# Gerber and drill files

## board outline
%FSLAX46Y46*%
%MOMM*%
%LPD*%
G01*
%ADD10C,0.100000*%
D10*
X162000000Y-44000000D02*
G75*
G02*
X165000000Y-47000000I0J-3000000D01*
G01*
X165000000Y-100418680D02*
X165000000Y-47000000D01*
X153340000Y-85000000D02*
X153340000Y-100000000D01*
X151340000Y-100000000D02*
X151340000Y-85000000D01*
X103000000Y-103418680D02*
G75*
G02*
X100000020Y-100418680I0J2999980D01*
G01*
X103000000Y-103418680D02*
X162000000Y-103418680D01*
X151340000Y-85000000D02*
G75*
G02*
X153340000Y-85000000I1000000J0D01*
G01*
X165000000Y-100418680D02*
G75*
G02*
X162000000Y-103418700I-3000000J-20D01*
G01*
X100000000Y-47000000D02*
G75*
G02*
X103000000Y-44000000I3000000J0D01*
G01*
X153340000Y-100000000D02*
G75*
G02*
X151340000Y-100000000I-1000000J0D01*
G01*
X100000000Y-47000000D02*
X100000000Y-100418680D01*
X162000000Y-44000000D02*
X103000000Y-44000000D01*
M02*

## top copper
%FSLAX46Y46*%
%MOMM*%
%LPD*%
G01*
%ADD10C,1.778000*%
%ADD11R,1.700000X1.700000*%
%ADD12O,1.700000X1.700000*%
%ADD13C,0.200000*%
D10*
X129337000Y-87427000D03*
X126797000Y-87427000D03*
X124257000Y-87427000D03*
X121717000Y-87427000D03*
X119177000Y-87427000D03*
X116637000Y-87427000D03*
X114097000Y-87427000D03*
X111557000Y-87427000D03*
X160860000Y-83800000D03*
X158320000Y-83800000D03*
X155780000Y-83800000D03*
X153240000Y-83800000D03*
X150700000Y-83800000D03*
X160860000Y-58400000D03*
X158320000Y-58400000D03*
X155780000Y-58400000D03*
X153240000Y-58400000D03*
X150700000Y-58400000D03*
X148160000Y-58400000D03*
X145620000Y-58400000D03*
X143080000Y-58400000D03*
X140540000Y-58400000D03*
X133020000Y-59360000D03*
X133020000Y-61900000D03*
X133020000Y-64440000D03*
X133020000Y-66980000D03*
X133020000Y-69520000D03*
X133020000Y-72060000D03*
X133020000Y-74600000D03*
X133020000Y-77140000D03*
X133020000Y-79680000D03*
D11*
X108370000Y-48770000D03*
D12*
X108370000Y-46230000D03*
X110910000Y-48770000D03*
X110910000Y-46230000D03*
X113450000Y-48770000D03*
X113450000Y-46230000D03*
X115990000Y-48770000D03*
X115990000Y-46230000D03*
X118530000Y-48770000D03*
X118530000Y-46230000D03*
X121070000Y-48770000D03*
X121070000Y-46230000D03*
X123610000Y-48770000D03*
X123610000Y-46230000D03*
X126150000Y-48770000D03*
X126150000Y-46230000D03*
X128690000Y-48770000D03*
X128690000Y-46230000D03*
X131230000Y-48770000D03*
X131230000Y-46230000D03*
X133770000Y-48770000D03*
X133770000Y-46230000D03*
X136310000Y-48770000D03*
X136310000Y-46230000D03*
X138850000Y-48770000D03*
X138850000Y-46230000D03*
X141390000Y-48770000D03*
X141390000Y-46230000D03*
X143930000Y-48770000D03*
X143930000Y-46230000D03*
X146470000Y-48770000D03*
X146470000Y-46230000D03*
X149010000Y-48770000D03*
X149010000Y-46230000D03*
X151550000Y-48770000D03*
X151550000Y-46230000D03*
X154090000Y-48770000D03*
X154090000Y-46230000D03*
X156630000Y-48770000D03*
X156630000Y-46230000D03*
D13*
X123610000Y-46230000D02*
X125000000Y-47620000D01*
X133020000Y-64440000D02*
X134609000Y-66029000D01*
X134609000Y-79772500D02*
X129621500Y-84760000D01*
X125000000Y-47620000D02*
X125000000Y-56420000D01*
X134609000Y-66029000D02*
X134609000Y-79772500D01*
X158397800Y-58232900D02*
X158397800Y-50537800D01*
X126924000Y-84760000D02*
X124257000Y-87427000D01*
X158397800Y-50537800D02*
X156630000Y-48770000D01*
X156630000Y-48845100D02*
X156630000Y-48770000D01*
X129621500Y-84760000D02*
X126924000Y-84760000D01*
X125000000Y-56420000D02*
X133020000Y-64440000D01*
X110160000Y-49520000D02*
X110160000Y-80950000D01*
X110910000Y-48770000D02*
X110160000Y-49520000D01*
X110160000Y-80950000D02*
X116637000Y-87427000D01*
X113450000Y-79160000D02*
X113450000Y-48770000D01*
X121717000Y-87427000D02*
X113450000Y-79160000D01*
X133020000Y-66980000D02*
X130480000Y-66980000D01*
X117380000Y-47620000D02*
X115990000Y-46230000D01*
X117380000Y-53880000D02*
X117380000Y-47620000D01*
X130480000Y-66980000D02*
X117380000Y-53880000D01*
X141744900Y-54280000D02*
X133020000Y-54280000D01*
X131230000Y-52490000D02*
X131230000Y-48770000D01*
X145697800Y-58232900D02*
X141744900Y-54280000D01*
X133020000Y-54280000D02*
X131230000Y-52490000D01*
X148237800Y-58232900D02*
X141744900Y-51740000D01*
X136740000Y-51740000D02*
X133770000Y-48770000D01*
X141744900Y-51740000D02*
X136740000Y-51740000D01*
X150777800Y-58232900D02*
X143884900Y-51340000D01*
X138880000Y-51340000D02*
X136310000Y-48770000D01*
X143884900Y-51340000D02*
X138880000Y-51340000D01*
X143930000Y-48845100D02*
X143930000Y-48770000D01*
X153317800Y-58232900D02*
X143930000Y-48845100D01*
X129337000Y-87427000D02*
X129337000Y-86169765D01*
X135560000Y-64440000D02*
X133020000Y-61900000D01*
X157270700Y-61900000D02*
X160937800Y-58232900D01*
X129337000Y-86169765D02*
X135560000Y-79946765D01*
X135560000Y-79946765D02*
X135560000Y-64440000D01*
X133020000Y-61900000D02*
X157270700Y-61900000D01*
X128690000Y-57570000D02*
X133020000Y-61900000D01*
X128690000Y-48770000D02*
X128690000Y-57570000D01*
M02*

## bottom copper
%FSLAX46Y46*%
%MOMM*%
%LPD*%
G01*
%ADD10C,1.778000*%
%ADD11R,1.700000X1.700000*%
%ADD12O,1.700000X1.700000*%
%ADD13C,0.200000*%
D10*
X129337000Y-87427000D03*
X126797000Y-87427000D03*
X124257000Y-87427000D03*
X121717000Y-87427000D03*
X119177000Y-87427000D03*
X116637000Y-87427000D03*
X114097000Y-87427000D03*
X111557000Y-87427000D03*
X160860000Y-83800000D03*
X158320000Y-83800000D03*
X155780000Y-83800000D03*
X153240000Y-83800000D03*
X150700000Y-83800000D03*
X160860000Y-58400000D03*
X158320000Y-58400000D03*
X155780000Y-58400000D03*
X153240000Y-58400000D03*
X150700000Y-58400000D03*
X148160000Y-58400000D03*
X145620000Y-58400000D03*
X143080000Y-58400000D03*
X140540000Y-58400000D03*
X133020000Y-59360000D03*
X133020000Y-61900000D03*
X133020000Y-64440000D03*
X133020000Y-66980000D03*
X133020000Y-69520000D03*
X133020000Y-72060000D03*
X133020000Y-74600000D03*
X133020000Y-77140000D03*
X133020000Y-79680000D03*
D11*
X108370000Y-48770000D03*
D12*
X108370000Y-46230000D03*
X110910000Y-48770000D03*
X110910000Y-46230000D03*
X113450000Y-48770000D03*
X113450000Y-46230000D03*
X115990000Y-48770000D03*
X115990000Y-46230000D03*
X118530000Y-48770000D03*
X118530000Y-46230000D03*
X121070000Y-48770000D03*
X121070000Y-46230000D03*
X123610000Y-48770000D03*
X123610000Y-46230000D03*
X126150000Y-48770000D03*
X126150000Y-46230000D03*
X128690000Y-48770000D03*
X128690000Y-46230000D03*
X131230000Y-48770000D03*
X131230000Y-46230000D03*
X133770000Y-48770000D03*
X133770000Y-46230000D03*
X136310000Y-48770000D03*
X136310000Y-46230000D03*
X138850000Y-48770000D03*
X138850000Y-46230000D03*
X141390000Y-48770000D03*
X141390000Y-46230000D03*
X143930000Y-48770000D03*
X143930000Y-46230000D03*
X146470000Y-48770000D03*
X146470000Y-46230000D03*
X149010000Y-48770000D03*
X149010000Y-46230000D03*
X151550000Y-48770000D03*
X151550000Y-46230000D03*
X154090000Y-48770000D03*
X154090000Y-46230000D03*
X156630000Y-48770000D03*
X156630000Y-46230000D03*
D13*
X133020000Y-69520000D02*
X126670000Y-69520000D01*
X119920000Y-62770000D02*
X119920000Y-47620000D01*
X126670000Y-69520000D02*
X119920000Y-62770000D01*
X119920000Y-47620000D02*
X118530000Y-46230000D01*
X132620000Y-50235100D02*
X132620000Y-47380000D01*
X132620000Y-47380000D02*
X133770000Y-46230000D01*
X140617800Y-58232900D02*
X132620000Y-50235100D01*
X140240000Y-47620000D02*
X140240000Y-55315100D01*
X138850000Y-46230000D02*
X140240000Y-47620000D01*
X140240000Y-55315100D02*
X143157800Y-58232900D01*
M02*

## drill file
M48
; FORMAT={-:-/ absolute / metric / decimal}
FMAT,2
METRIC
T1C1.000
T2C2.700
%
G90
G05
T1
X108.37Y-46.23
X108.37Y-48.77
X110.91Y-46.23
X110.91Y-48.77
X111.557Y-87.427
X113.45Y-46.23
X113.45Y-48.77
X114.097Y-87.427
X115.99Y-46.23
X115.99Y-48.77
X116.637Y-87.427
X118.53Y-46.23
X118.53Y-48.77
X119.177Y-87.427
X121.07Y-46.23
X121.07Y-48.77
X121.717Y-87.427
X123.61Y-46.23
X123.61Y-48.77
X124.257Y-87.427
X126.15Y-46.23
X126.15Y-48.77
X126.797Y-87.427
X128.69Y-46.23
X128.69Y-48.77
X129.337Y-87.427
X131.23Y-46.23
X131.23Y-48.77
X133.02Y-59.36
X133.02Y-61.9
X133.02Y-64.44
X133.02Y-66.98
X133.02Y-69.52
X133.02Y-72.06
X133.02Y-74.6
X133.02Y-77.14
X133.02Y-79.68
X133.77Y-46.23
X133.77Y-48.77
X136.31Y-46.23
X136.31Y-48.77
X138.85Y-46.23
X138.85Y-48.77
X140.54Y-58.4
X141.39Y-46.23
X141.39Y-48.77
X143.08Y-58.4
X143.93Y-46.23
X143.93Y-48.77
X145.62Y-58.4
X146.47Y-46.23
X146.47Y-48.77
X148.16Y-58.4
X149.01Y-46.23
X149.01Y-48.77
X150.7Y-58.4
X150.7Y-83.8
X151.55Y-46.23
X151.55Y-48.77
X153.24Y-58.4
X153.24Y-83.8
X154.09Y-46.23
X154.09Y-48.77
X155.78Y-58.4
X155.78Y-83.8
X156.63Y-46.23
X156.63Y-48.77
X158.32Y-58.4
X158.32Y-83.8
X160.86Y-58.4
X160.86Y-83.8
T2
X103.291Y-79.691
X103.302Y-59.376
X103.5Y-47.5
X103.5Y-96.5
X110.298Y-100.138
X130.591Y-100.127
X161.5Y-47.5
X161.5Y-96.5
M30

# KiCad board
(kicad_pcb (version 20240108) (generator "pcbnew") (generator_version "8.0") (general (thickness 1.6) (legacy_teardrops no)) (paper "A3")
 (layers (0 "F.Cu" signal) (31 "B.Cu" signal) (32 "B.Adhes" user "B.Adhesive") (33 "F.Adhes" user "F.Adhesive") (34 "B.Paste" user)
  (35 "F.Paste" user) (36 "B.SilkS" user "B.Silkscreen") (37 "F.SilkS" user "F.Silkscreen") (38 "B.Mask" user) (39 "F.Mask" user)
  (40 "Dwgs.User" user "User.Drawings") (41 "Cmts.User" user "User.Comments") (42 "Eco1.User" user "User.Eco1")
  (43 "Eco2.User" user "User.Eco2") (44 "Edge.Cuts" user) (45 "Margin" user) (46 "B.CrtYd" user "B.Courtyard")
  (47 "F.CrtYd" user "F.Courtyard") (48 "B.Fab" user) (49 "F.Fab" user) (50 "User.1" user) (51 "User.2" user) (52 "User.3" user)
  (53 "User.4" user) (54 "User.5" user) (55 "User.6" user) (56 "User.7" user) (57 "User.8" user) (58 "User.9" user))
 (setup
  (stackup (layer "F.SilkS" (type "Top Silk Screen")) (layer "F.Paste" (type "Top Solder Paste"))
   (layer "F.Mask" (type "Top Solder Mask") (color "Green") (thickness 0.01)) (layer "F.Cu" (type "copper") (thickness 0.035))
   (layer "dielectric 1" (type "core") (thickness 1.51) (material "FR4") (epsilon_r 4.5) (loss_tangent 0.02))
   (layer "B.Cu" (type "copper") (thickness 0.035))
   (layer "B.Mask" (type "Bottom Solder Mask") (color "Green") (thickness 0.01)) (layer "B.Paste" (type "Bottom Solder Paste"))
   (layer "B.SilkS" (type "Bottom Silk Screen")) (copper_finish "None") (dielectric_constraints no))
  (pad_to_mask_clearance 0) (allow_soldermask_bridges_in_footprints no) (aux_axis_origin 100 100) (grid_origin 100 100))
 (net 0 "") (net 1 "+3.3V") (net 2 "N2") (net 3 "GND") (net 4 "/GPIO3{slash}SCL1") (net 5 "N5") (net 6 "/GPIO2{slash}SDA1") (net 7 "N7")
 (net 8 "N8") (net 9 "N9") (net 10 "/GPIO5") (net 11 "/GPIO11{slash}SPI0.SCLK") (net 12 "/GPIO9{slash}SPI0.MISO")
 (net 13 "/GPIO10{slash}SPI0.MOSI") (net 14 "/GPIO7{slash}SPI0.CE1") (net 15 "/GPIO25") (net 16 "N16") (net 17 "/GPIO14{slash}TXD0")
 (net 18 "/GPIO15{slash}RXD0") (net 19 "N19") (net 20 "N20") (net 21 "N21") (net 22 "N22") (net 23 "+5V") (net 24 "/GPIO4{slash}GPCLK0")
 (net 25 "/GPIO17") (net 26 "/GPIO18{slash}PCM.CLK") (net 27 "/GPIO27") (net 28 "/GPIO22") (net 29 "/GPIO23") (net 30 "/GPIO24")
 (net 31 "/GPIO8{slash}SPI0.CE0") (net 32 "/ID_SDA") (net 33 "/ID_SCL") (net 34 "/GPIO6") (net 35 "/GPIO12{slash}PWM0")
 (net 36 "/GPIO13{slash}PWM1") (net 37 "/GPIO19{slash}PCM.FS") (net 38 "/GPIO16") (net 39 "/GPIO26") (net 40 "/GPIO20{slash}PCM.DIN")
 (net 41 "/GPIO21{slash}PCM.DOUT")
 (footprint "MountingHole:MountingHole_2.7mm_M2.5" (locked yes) (layer "F.Cu") (at 161.5 47.5)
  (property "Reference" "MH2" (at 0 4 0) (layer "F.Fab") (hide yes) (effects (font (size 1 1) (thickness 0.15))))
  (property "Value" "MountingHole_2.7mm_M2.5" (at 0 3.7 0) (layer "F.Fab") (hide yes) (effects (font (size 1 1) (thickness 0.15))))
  (pad "" np_thru_hole circle (at 0 0) (size 2.7 2.7) (drill 2.7) (layers "*.Cu" "*.Mask")))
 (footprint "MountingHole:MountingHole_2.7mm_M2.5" (layer "F.Cu") (at 103.290686 79.691314)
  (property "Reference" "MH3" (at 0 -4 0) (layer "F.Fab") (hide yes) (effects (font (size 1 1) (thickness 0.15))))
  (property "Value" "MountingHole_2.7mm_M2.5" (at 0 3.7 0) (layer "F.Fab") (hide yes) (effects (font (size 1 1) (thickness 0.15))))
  (pad "" np_thru_hole circle (at 0 0) (size 2.7 2.7) (drill 2.7) (layers "*.Cu" "*.Mask")))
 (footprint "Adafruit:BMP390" (layer "F.Cu") (at 120.32 92.38 180)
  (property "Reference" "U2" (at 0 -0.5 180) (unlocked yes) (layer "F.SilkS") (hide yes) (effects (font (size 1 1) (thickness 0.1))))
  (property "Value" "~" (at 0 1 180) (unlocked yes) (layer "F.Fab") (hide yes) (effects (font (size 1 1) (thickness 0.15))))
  (pad "1" thru_hole circle (at -9.017 4.953 270) (size 1.778 1.778) (drill 1) (layers "*.Cu" "*.Mask") (remove_unused_layers no)
   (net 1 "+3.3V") (solder_mask_margin 0.0508) (thermal_bridge_angle 0))
  (pad "2" thru_hole circle (at -6.477 4.953 270) (size 1.778 1.778) (drill 1) (layers "*.Cu" "*.Mask") (remove_unused_layers no)
   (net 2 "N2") (solder_mask_margin 0.0508) (thermal_bridge_angle 0))
  (pad "3" thru_hole circle (at -3.937 4.953 270) (size 1.778 1.778) (drill 1) (layers "*.Cu" "*.Mask") (remove_unused_layers no)
   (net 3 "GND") (solder_mask_margin 0.0508) (thermal_bridge_angle 0))
  (pad "4" thru_hole circle (at -1.397 4.953 270) (size 1.778 1.778) (drill 1) (layers "*.Cu" "*.Mask") (remove_unused_layers no)
   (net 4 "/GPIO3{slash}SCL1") (solder_mask_margin 0.0508) (thermal_bridge_angle 0))
  (pad "5" thru_hole circle (at 1.143 4.953 270) (size 1.778 1.778) (drill 1) (layers "*.Cu" "*.Mask") (remove_unused_layers no)
   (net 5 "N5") (solder_mask_margin 0.0508) (thermal_bridge_angle 0))
  (pad "6" thru_hole circle (at 3.683 4.953 270) (size 1.778 1.778) (drill 1) (layers "*.Cu" "*.Mask") (remove_unused_layers no)
   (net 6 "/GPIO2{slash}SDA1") (solder_mask_margin 0.0508) (thermal_bridge_angle 0))
  (pad "7" thru_hole circle (at 6.223 4.953 270) (size 1.778 1.778) (drill 1) (layers "*.Cu" "*.Mask") (remove_unused_layers no)
   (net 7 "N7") (solder_mask_margin 0.0508) (thermal_bridge_angle 0))
  (pad "8" thru_hole circle (at 8.763 4.953 270) (size 1.778 1.778) (drill 1) (layers "*.Cu" "*.Mask") (remove_unused_layers no)
   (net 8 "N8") (solder_mask_margin 0.0508) (thermal_bridge_angle 0)))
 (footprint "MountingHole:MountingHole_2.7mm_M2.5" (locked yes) (layer "F.Cu") (at 103.5 96.5)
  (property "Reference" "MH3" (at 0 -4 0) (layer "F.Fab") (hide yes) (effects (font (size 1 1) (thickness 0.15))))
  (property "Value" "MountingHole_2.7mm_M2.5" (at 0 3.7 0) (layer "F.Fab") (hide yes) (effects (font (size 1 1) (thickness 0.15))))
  (pad "" np_thru_hole circle (at 0 0) (size 2.7 2.7) (drill 2.7) (layers "*.Cu" "*.Mask")))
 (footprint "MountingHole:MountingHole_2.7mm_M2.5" (layer "F.Cu") (at 130.591 100.127)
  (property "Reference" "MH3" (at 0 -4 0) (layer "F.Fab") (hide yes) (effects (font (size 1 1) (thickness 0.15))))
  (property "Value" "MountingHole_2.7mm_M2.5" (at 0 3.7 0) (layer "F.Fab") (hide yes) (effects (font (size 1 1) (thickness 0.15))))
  (pad "" np_thru_hole circle (at 0 0) (size 2.7 2.7) (drill 2.7) (layers "*.Cu" "*.Mask")))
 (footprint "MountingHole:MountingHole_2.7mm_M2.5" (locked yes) (layer "F.Cu") (at 103.5 47.5)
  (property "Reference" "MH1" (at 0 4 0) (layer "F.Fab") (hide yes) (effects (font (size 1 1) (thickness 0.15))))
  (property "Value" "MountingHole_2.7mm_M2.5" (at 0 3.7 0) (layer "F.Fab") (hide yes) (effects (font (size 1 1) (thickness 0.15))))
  (pad "" np_thru_hole circle (at 0 0) (size 2.7 2.7) (drill 2.7) (layers "*.Cu" "*.Mask")))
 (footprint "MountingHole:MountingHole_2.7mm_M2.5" (layer "F.Cu") (at 110.298314 100.138314)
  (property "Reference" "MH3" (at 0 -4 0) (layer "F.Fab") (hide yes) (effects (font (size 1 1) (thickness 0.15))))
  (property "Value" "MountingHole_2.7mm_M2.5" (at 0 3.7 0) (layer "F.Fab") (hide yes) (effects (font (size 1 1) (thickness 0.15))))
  (pad "" np_thru_hole circle (at 0 0) (size 2.7 2.7) (drill 2.7) (layers "*.Cu" "*.Mask")))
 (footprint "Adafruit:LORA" (layer "F.Cu") (at 150.7222 69.6871 180)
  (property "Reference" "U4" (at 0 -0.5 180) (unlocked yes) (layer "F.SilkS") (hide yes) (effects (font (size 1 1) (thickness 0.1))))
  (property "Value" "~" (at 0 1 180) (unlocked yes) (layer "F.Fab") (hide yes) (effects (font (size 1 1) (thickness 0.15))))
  (pad "" thru_hole circle (at -10.1378 -14.1129 270) (size 1.778 1.778) (drill 1) (layers "*.Cu" "*.Mask") (remove_unused_layers no)
   (solder_mask_margin 0.0508) (thermal_bridge_angle 0))
  (pad "" thru_hole circle (at -7.5978 -14.1129 270) (size 1.778 1.778) (drill 1) (layers "*.Cu" "*.Mask") (remove_unused_layers no)
   (solder_mask_margin 0.0508) (thermal_bridge_angle 0))
  (pad "" thru_hole circle (at -5.0578 -14.1129 270) (size 1.778 1.778) (drill 1) (layers "*.Cu" "*.Mask") (remove_unused_layers no)
   (solder_mask_margin 0.0508) (thermal_bridge_angle 0))
  (pad "" thru_hole circle (at -2.5178 -14.1129 270) (size 1.778 1.778) (drill 1) (layers "*.Cu" "*.Mask") (remove_unused_layers no)
   (solder_mask_margin 0.0508) (thermal_bridge_angle 0))
  (pad "" thru_hole circle (at 0.0222 -14.1129 270) (size 1.778 1.778) (drill 1) (layers "*.Cu" "*.Mask") (remove_unused_layers no)
   (solder_mask_margin 0.0508) (thermal_bridge_angle 0))
  (pad "1" thru_hole circle (at -10.1378 11.2871 270) (size 1.778 1.778) (drill 1) (layers "*.Cu" "*.Mask") (remove_unused_layers no)
   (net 1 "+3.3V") (solder_mask_margin 0.0508) (thermal_bridge_angle 0))
  (pad "2" thru_hole circle (at -7.5978 11.2871 270) (size 1.778 1.778) (drill 1) (layers "*.Cu" "*.Mask") (remove_unused_layers no)
   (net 3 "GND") (solder_mask_margin 0.0508) (thermal_bridge_angle 0))
  (pad "3" thru_hole circle (at -5.0578 11.2871 270) (size 1.778 1.778) (drill 1) (layers "*.Cu" "*.Mask") (remove_unused_layers no)
   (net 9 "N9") (solder_mask_margin 0.0508) (thermal_bridge_angle 0))
  (pad "4" thru_hole circle (at -2.5178 11.2871 270) (size 1.778 1.778) (drill 1) (layers "*.Cu" "*.Mask") (remove_unused_layers no)
   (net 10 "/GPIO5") (solder_mask_margin 0.0508) (thermal_bridge_angle 0))
  (pad "5" thru_hole circle (at 0.0222 11.2871 270) (size 1.778 1.778) (drill 1) (layers "*.Cu" "*.Mask") (remove_unused_layers no)
   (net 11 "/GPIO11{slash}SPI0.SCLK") (solder_mask_margin 0.0508) (thermal_bridge_angle 0))
  (pad "6" thru_hole circle (at 2.5622 11.2871 270) (size 1.778 1.778) (drill 1) (layers "*.Cu" "*.Mask") (remove_unused_layers no)
   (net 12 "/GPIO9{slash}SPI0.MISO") (solder_mask_margin 0.0508) (thermal_bridge_angle 0))
  (pad "7" thru_hole circle (at 5.1022 11.2871 270) (size 1.778 1.778) (drill 1) (layers "*.Cu" "*.Mask") (remove_unused_layers no)
   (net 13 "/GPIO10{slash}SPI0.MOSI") (solder_mask_margin 0.0508) (thermal_bridge_angle 0))
  (pad "8" thru_hole circle (at 7.6422 11.2871 270) (size 1.778 1.778) (drill 1) (layers "*.Cu" "*.Mask") (remove_unused_layers no)
   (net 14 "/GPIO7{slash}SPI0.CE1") (solder_mask_margin 0.0508) (thermal_bridge_angle 0))
  (pad "9" thru_hole circle (at 10.1822 11.2871 270) (size 1.778 1.778) (drill 1) (layers "*.Cu" "*.Mask") (remove_unused_layers no)
   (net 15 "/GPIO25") (solder_mask_margin 0.0508) (thermal_bridge_angle 0)))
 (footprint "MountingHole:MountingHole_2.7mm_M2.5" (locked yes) (layer "F.Cu") (at 161.5 96.5)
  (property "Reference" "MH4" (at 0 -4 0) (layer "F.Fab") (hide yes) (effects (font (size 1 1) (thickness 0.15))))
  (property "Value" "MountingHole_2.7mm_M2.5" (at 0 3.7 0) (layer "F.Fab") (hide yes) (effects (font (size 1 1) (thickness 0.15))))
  (pad "" np_thru_hole circle (at 0 0) (size 2.7 2.7) (drill 2.7) (layers "*.Cu" "*.Mask")))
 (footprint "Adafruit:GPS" (layer "F.Cu") (at 132.639 69.393 90)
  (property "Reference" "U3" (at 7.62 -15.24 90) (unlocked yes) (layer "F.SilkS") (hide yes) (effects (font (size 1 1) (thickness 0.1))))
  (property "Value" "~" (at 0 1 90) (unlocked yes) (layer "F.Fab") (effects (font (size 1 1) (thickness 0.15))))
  (pad "1" thru_hole circle (at 10.033 0.381) (size 1.778 1.778) (drill 1) (layers "*.Cu" "*.Mask") (remove_unused_layers no) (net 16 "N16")
   (solder_mask_margin 0.0508) (thermal_bridge_angle 0))
  (pad "2" thru_hole circle (at 7.493 0.381) (size 1.778 1.778) (drill 1) (layers "*.Cu" "*.Mask") (remove_unused_layers no) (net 1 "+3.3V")
   (solder_mask_margin 0.0508) (thermal_bridge_angle 0))
  (pad "3" thru_hole circle (at 4.953 0.381) (size 1.778 1.778) (drill 1) (layers "*.Cu" "*.Mask") (remove_unused_layers no) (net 3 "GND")
   (solder_mask_margin 0.0508) (thermal_bridge_angle 0))
  (pad "4" thru_hole circle (at 2.413 0.381) (size 1.778 1.778) (drill 1) (layers "*.Cu" "*.Mask") (remove_unused_layers no)
   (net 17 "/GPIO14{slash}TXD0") (solder_mask_margin 0.0508) (thermal_bridge_angle 0))
  (pad "5" thru_hole circle (at -0.127 0.381) (size 1.778 1.778) (drill 1) (layers "*.Cu" "*.Mask") (remove_unused_layers no)
   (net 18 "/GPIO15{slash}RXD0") (solder_mask_margin 0.0508) (thermal_bridge_angle 0))
  (pad "6" thru_hole circle (at -2.667 0.381) (size 1.778 1.778) (drill 1) (layers "*.Cu" "*.Mask") (remove_unused_layers no) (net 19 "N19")
   (solder_mask_margin 0.0508) (thermal_bridge_angle 0))
  (pad "7" thru_hole circle (at -5.207 0.381) (size 1.778 1.778) (drill 1) (layers "*.Cu" "*.Mask") (remove_unused_layers no) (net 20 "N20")
   (solder_mask_margin 0.0508) (thermal_bridge_angle 0))
  (pad "8" thru_hole circle (at -7.747 0.381) (size 1.778 1.778) (drill 1) (layers "*.Cu" "*.Mask") (remove_unused_layers no) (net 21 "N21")
   (solder_mask_margin 0.0508) (thermal_bridge_angle 0))
  (pad "9" thru_hole circle (at -10.287 0.381) (size 1.778 1.778) (drill 1) (layers "*.Cu" "*.Mask") (remove_unused_layers no)
   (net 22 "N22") (solder_mask_margin 0.0508) (thermal_bridge_angle 0)))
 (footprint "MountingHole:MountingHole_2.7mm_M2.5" (layer "F.Cu") (at 103.302 59.376)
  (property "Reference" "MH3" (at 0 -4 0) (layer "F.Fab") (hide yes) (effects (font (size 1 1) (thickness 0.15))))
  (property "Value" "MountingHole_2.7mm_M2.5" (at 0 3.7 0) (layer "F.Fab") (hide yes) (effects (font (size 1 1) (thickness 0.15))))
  (pad "" np_thru_hole circle (at 0 0) (size 2.7 2.7) (drill 2.7) (layers "*.Cu" "*.Mask")))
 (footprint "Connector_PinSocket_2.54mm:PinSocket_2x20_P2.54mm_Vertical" (layer "B.Cu") (at 108.37 48.77 -90)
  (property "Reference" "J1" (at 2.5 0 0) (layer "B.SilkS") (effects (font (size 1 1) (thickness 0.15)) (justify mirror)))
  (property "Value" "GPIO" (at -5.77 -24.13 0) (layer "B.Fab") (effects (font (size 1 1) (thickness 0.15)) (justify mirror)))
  (pad "1" thru_hole rect (at 0 0 270) (size 1.7 1.7) (drill 1) (layers "*.Cu" "*.Mask") (remove_unused_layers no) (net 1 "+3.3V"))
  (pad "2" thru_hole oval (at -2.54 0 270) (size 1.7 1.7) (drill 1) (layers "*.Cu" "*.Mask") (remove_unused_layers no) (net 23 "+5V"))
  (pad "3" thru_hole oval (at 0 -2.54 270) (size 1.7 1.7) (drill 1) (layers "*.Cu" "*.Mask") (remove_unused_layers no)
   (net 6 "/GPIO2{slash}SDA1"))
  (pad "4" thru_hole oval (at -2.54 -2.54 270) (size 1.7 1.7) (drill 1) (layers "*.Cu" "*.Mask") (remove_unused_layers no) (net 23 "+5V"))
  (pad "5" thru_hole oval (at 0 -5.08 270) (size 1.7 1.7) (drill 1) (layers "*.Cu" "*.Mask") (remove_unused_layers no)
   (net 4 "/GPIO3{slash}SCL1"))
  (pad "6" thru_hole oval (at -2.54 -5.08 270) (size 1.7 1.7) (drill 1) (layers "*.Cu" "*.Mask") (remove_unused_layers no) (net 3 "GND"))
  (pad "7" thru_hole oval (at 0 -7.62 270) (size 1.7 1.7) (drill 1) (layers "*.Cu" "*.Mask") (remove_unused_layers no)
   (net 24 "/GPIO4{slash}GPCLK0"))
  (pad "8" thru_hole oval (at -2.54 -7.62 270) (size 1.7 1.7) (drill 1) (layers "*.Cu" "*.Mask") (remove_unused_layers no)
   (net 17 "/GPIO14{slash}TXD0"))
  (pad "9" thru_hole oval (at 0 -10.16 270) (size 1.7 1.7) (drill 1) (layers "*.Cu" "*.Mask") (remove_unused_layers no) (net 3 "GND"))
  (pad "10" thru_hole oval (at -2.54 -10.16 270) (size 1.7 1.7) (drill 1) (layers "*.Cu" "*.Mask") (remove_unused_layers no)
   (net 18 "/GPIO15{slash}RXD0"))
  (pad "11" thru_hole oval (at 0 -12.7 270) (size 1.7 1.7) (drill 1) (layers "*.Cu" "*.Mask") (remove_unused_layers no) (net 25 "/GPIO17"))
  (pad "12" thru_hole oval (at -2.54 -12.7 270) (size 1.7 1.7) (drill 1) (layers "*.Cu" "*.Mask") (remove_unused_layers no)
   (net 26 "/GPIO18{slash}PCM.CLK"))
  (pad "13" thru_hole oval (at 0 -15.24 270) (size 1.7 1.7) (drill 1) (layers "*.Cu" "*.Mask") (remove_unused_layers no) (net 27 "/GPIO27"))
  (pad "14" thru_hole oval (at -2.54 -15.24 270) (size 1.7 1.7) (drill 1) (layers "*.Cu" "*.Mask") (remove_unused_layers no) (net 3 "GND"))
  (pad "15" thru_hole oval (at 0 -17.78 270) (size 1.7 1.7) (drill 1) (layers "*.Cu" "*.Mask") (remove_unused_layers no) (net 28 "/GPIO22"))
  (pad "16" thru_hole oval (at -2.54 -17.78 270) (size 1.7 1.7) (drill 1) (layers "*.Cu" "*.Mask") (remove_unused_layers no)
   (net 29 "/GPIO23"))
  (pad "17" thru_hole oval (at 0 -20.32 270) (size 1.7 1.7) (drill 1) (layers "*.Cu" "*.Mask") (remove_unused_layers no) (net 1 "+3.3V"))
  (pad "18" thru_hole oval (at -2.54 -20.32 270) (size 1.7 1.7) (drill 1) (layers "*.Cu" "*.Mask") (remove_unused_layers no)
   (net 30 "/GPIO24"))
  (pad "19" thru_hole oval (at 0 -22.86 270) (size 1.7 1.7) (drill 1) (layers "*.Cu" "*.Mask") (remove_unused_layers no)
   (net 13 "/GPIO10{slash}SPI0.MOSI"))
  (pad "20" thru_hole oval (at -2.54 -22.86 270) (size 1.7 1.7) (drill 1) (layers "*.Cu" "*.Mask") (remove_unused_layers no) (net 3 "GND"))
  (pad "21" thru_hole oval (at 0 -25.4 270) (size 1.7 1.7) (drill 1) (layers "*.Cu" "*.Mask") (remove_unused_layers no)
   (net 12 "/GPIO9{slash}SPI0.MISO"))
  (pad "22" thru_hole oval (at -2.54 -25.4 270) (size 1.7 1.7) (drill 1) (layers "*.Cu" "*.Mask") (remove_unused_layers no)
   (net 15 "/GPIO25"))
  (pad "23" thru_hole oval (at 0 -27.94 270) (size 1.7 1.7) (drill 1) (layers "*.Cu" "*.Mask") (remove_unused_layers no)
   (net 11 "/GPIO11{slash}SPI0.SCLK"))
  (pad "24" thru_hole oval (at -2.54 -27.94 270) (size 1.7 1.7) (drill 1) (layers "*.Cu" "*.Mask") (remove_unused_layers no)
   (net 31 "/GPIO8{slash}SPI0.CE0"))
  (pad "25" thru_hole oval (at 0 -30.48 270) (size 1.7 1.7) (drill 1) (layers "*.Cu" "*.Mask") (remove_unused_layers no) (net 3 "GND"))
  (pad "26" thru_hole oval (at -2.54 -30.48 270) (size 1.7 1.7) (drill 1) (layers "*.Cu" "*.Mask") (remove_unused_layers no)
   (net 14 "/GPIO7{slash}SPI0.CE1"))
  (pad "27" thru_hole oval (at 0 -33.02 270) (size 1.7 1.7) (drill 1) (layers "*.Cu" "*.Mask") (remove_unused_layers no) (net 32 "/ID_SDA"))
  (pad "28" thru_hole oval (at -2.54 -33.02 270) (size 1.7 1.7) (drill 1) (layers "*.Cu" "*.Mask") (remove_unused_layers no)
   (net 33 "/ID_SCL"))
  (pad "29" thru_hole oval (at 0 -35.56 270) (size 1.7 1.7) (drill 1) (layers "*.Cu" "*.Mask") (remove_unused_layers no) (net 10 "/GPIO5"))
  (pad "30" thru_hole oval (at -2.54 -35.56 270) (size 1.7 1.7) (drill 1) (layers "*.Cu" "*.Mask") (remove_unused_layers no) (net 3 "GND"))
  (pad "31" thru_hole oval (at 0 -38.1 270) (size 1.7 1.7) (drill 1) (layers "*.Cu" "*.Mask") (remove_unused_layers no) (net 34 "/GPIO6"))
  (pad "32" thru_hole oval (at -2.54 -38.1 270) (size 1.7 1.7) (drill 1) (layers "*.Cu" "*.Mask") (remove_unused_layers no)
   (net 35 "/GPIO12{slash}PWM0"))
  (pad "33" thru_hole oval (at 0 -40.64 270) (size 1.7 1.7) (drill 1) (layers "*.Cu" "*.Mask") (remove_unused_layers no)
   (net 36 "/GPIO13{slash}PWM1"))
  (pad "34" thru_hole oval (at -2.54 -40.64 270) (size 1.7 1.7) (drill 1) (layers "*.Cu" "*.Mask") (remove_unused_layers no) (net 3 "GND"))
  (pad "35" thru_hole oval (at 0 -43.18 270) (size 1.7 1.7) (drill 1) (layers "*.Cu" "*.Mask") (remove_unused_layers no)
   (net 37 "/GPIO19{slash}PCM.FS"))
  (pad "36" thru_hole oval (at -2.54 -43.18 270) (size 1.7 1.7) (drill 1) (layers "*.Cu" "*.Mask") (remove_unused_layers no)
   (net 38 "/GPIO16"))
  (pad "37" thru_hole oval (at 0 -45.72 270) (size 1.7 1.7) (drill 1) (layers "*.Cu" "*.Mask") (remove_unused_layers no) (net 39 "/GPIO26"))
  (pad "38" thru_hole oval (at -2.54 -45.72 270) (size 1.7 1.7) (drill 1) (layers "*.Cu" "*.Mask") (remove_unused_layers no)
   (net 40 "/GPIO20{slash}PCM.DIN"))
  (pad "39" thru_hole oval (at 0 -48.26 270) (size 1.7 1.7) (drill 1) (layers "*.Cu" "*.Mask") (remove_unused_layers no) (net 3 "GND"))
  (pad "40" thru_hole oval (at -2.54 -48.26 270) (size 1.7 1.7) (drill 1) (layers "*.Cu" "*.Mask") (remove_unused_layers no)
   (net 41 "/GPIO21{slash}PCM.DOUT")))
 (gr_arc (start 162 44) (mid 164.12132 44.87868) (end 165 47) (stroke (width 0.1) (type solid)) (layer "Edge.Cuts"))
 (gr_line (start 165 100.41868) (end 165 47) (stroke (width 0.1) (type solid)) (layer "Edge.Cuts"))
 (gr_line (start 153.34 85) (end 153.34 100) (stroke (width 0.1) (type solid)) (layer "Edge.Cuts"))
 (gr_line (start 151.34 100) (end 151.34 85) (stroke (width 0.1) (type solid)) (layer "Edge.Cuts"))
 (gr_arc (start 103 103.41868) (mid 100.87868 102.54) (end 100 100.41868) (stroke (width 0.1) (type solid)) (layer "Edge.Cuts"))
 (gr_line (start 103 103.41868) (end 162 103.41868) (stroke (width 0.1) (type solid)) (layer "Edge.Cuts"))
 (gr_arc (start 151.34 85) (mid 152.34 84) (end 153.34 85) (stroke (width 0.1) (type solid)) (layer "Edge.Cuts"))
 (gr_arc (start 165 100.41868) (mid 164.12132 102.54) (end 162 103.41868) (stroke (width 0.1) (type solid)) (layer "Edge.Cuts"))
 (gr_arc (start 100 47) (mid 100.87868 44.87868) (end 103 44) (stroke (width 0.1) (type solid)) (layer "Edge.Cuts"))
 (gr_arc (start 153.34 100) (mid 152.34 101) (end 151.34 100) (stroke (width 0.1) (type solid)) (layer "Edge.Cuts"))
 (gr_line (start 100 47) (end 100 100.41868) (stroke (width 0.1) (type solid)) (layer "Edge.Cuts"))
 (gr_line (start 162 44) (end 103 44) (stroke (width 0.1) (type solid)) (layer "Edge.Cuts"))
 (segment (start 123.61 46.23) (end 125 47.62) (width 0.2) (layer "F.Cu") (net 3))
 (segment (start 133.02 64.44) (end 134.609 66.029) (width 0.2) (layer "F.Cu") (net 3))
 (segment (start 134.609 79.7725) (end 129.6215 84.76) (width 0.2) (layer "F.Cu") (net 3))
 (segment (start 125 47.62) (end 125 56.42) (width 0.2) (layer "F.Cu") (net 3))
 (segment (start 134.609 66.029) (end 134.609 79.7725) (width 0.2) (layer "F.Cu") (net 3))
 (segment (start 158.3978 58.2329) (end 158.3978 50.5378) (width 0.2) (layer "F.Cu") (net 3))
 (segment (start 126.924 84.76) (end 124.257 87.427) (width 0.2) (layer "F.Cu") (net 3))
 (segment (start 158.3978 50.5378) (end 156.63 48.77) (width 0.2) (layer "F.Cu") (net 3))
 (segment (start 156.63 48.8451) (end 156.63 48.77) (width 0.2) (layer "F.Cu") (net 3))
 (segment (start 129.6215 84.76) (end 126.924 84.76) (width 0.2) (layer "F.Cu") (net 3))
 (segment (start 125 56.42) (end 133.02 64.44) (width 0.2) (layer "F.Cu") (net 3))
 (segment (start 110.16 49.52) (end 110.16 80.95) (width 0.2) (layer "F.Cu") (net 6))
 (segment (start 110.91 48.77) (end 110.16 49.52) (width 0.2) (layer "F.Cu") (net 6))
 (segment (start 110.16 80.95) (end 116.637 87.427) (width 0.2) (layer "F.Cu") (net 6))
 (segment (start 113.45 79.16) (end 113.45 48.77) (width 0.2) (layer "F.Cu") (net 4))
 (segment (start 121.717 87.427) (end 113.45 79.16) (width 0.2) (layer "F.Cu") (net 4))
 (segment (start 133.02 66.98) (end 130.48 66.98) (width 0.2) (layer "F.Cu") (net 17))
 (segment (start 117.38 47.62) (end 115.99 46.23) (width 0.2) (layer "F.Cu") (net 17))
 (segment (start 117.38 53.88) (end 117.38 47.62) (width 0.2) (layer "F.Cu") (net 17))
 (segment (start 130.48 66.98) (end 117.38 53.88) (width 0.2) (layer "F.Cu") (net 17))
 (segment (start 133.02 69.52) (end 126.67 69.52) (width 0.2) (layer "B.Cu") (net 18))
 (segment (start 119.92 62.77) (end 119.92 47.62) (width 0.2) (layer "B.Cu") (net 18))
 (segment (start 126.67 69.52) (end 119.92 62.77) (width 0.2) (layer "B.Cu") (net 18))
 (segment (start 119.92 47.62) (end 118.53 46.23) (width 0.2) (layer "B.Cu") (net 18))
 (segment (start 141.7449 54.28) (end 133.02 54.28) (width 0.2) (layer "F.Cu") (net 13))
 (segment (start 131.23 52.49) (end 131.23 48.77) (width 0.2) (layer "F.Cu") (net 13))
 (segment (start 145.6978 58.2329) (end 141.7449 54.28) (width 0.2) (layer "F.Cu") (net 13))
 (segment (start 133.02 54.28) (end 131.23 52.49) (width 0.2) (layer "F.Cu") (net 13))
 (segment (start 148.2378 58.2329) (end 141.7449 51.74) (width 0.2) (layer "F.Cu") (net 12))
 (segment (start 136.74 51.74) (end 133.77 48.77) (width 0.2) (layer "F.Cu") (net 12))
 (segment (start 141.7449 51.74) (end 136.74 51.74) (width 0.2) (layer "F.Cu") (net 12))
 (segment (start 132.62 50.2351) (end 132.62 47.38) (width 0.2) (layer "B.Cu") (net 15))
 (segment (start 132.62 47.38) (end 133.77 46.23) (width 0.2) (layer "B.Cu") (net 15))
 (segment (start 140.6178 58.2329) (end 132.62 50.2351) (width 0.2) (layer "B.Cu") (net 15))
 (segment (start 150.7778 58.2329) (end 143.8849 51.34) (width 0.2) (layer "F.Cu") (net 11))
 (segment (start 138.88 51.34) (end 136.31 48.77) (width 0.2) (layer "F.Cu") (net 11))
 (segment (start 143.8849 51.34) (end 138.88 51.34) (width 0.2) (layer "F.Cu") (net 11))
 (segment (start 140.24 47.62) (end 140.24 55.3151) (width 0.2) (layer "B.Cu") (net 14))
 (segment (start 138.85 46.23) (end 140.24 47.62) (width 0.2) (layer "B.Cu") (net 14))
 (segment (start 140.24 55.3151) (end 143.1578 58.2329) (width 0.2) (layer "B.Cu") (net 14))
 (segment (start 143.93 48.8451) (end 143.93 48.77) (width 0.2) (layer "F.Cu") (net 10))
 (segment (start 153.3178 58.2329) (end 143.93 48.8451) (width 0.2) (layer "F.Cu") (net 10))
 (segment (start 129.337 87.427) (end 129.337 86.169765) (width 0.2) (layer "F.Cu") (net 1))
 (segment (start 135.56 64.44) (end 133.02 61.9) (width 0.2) (layer "F.Cu") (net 1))
 (segment (start 157.2707 61.9) (end 160.9378 58.2329) (width 0.2) (layer "F.Cu") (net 1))
 (segment (start 129.337 86.169765) (end 135.56 79.946765) (width 0.2) (layer "F.Cu") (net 1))
 (segment (start 135.56 79.946765) (end 135.56 64.44) (width 0.2) (layer "F.Cu") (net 1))
 (segment (start 133.02 61.9) (end 157.2707 61.9) (width 0.2) (layer "F.Cu") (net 1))
 (segment (start 128.69 57.57) (end 133.02 61.9) (width 0.2) (layer "F.Cu") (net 1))
 (segment (start 128.69 48.77) (end 128.69 57.57) (width 0.2) (layer "F.Cu") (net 1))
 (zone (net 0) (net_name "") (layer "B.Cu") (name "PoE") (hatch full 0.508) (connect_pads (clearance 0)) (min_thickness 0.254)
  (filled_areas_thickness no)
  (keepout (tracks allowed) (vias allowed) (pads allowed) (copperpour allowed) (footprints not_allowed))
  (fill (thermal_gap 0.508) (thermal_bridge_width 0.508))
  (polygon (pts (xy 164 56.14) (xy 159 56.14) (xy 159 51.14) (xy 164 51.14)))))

